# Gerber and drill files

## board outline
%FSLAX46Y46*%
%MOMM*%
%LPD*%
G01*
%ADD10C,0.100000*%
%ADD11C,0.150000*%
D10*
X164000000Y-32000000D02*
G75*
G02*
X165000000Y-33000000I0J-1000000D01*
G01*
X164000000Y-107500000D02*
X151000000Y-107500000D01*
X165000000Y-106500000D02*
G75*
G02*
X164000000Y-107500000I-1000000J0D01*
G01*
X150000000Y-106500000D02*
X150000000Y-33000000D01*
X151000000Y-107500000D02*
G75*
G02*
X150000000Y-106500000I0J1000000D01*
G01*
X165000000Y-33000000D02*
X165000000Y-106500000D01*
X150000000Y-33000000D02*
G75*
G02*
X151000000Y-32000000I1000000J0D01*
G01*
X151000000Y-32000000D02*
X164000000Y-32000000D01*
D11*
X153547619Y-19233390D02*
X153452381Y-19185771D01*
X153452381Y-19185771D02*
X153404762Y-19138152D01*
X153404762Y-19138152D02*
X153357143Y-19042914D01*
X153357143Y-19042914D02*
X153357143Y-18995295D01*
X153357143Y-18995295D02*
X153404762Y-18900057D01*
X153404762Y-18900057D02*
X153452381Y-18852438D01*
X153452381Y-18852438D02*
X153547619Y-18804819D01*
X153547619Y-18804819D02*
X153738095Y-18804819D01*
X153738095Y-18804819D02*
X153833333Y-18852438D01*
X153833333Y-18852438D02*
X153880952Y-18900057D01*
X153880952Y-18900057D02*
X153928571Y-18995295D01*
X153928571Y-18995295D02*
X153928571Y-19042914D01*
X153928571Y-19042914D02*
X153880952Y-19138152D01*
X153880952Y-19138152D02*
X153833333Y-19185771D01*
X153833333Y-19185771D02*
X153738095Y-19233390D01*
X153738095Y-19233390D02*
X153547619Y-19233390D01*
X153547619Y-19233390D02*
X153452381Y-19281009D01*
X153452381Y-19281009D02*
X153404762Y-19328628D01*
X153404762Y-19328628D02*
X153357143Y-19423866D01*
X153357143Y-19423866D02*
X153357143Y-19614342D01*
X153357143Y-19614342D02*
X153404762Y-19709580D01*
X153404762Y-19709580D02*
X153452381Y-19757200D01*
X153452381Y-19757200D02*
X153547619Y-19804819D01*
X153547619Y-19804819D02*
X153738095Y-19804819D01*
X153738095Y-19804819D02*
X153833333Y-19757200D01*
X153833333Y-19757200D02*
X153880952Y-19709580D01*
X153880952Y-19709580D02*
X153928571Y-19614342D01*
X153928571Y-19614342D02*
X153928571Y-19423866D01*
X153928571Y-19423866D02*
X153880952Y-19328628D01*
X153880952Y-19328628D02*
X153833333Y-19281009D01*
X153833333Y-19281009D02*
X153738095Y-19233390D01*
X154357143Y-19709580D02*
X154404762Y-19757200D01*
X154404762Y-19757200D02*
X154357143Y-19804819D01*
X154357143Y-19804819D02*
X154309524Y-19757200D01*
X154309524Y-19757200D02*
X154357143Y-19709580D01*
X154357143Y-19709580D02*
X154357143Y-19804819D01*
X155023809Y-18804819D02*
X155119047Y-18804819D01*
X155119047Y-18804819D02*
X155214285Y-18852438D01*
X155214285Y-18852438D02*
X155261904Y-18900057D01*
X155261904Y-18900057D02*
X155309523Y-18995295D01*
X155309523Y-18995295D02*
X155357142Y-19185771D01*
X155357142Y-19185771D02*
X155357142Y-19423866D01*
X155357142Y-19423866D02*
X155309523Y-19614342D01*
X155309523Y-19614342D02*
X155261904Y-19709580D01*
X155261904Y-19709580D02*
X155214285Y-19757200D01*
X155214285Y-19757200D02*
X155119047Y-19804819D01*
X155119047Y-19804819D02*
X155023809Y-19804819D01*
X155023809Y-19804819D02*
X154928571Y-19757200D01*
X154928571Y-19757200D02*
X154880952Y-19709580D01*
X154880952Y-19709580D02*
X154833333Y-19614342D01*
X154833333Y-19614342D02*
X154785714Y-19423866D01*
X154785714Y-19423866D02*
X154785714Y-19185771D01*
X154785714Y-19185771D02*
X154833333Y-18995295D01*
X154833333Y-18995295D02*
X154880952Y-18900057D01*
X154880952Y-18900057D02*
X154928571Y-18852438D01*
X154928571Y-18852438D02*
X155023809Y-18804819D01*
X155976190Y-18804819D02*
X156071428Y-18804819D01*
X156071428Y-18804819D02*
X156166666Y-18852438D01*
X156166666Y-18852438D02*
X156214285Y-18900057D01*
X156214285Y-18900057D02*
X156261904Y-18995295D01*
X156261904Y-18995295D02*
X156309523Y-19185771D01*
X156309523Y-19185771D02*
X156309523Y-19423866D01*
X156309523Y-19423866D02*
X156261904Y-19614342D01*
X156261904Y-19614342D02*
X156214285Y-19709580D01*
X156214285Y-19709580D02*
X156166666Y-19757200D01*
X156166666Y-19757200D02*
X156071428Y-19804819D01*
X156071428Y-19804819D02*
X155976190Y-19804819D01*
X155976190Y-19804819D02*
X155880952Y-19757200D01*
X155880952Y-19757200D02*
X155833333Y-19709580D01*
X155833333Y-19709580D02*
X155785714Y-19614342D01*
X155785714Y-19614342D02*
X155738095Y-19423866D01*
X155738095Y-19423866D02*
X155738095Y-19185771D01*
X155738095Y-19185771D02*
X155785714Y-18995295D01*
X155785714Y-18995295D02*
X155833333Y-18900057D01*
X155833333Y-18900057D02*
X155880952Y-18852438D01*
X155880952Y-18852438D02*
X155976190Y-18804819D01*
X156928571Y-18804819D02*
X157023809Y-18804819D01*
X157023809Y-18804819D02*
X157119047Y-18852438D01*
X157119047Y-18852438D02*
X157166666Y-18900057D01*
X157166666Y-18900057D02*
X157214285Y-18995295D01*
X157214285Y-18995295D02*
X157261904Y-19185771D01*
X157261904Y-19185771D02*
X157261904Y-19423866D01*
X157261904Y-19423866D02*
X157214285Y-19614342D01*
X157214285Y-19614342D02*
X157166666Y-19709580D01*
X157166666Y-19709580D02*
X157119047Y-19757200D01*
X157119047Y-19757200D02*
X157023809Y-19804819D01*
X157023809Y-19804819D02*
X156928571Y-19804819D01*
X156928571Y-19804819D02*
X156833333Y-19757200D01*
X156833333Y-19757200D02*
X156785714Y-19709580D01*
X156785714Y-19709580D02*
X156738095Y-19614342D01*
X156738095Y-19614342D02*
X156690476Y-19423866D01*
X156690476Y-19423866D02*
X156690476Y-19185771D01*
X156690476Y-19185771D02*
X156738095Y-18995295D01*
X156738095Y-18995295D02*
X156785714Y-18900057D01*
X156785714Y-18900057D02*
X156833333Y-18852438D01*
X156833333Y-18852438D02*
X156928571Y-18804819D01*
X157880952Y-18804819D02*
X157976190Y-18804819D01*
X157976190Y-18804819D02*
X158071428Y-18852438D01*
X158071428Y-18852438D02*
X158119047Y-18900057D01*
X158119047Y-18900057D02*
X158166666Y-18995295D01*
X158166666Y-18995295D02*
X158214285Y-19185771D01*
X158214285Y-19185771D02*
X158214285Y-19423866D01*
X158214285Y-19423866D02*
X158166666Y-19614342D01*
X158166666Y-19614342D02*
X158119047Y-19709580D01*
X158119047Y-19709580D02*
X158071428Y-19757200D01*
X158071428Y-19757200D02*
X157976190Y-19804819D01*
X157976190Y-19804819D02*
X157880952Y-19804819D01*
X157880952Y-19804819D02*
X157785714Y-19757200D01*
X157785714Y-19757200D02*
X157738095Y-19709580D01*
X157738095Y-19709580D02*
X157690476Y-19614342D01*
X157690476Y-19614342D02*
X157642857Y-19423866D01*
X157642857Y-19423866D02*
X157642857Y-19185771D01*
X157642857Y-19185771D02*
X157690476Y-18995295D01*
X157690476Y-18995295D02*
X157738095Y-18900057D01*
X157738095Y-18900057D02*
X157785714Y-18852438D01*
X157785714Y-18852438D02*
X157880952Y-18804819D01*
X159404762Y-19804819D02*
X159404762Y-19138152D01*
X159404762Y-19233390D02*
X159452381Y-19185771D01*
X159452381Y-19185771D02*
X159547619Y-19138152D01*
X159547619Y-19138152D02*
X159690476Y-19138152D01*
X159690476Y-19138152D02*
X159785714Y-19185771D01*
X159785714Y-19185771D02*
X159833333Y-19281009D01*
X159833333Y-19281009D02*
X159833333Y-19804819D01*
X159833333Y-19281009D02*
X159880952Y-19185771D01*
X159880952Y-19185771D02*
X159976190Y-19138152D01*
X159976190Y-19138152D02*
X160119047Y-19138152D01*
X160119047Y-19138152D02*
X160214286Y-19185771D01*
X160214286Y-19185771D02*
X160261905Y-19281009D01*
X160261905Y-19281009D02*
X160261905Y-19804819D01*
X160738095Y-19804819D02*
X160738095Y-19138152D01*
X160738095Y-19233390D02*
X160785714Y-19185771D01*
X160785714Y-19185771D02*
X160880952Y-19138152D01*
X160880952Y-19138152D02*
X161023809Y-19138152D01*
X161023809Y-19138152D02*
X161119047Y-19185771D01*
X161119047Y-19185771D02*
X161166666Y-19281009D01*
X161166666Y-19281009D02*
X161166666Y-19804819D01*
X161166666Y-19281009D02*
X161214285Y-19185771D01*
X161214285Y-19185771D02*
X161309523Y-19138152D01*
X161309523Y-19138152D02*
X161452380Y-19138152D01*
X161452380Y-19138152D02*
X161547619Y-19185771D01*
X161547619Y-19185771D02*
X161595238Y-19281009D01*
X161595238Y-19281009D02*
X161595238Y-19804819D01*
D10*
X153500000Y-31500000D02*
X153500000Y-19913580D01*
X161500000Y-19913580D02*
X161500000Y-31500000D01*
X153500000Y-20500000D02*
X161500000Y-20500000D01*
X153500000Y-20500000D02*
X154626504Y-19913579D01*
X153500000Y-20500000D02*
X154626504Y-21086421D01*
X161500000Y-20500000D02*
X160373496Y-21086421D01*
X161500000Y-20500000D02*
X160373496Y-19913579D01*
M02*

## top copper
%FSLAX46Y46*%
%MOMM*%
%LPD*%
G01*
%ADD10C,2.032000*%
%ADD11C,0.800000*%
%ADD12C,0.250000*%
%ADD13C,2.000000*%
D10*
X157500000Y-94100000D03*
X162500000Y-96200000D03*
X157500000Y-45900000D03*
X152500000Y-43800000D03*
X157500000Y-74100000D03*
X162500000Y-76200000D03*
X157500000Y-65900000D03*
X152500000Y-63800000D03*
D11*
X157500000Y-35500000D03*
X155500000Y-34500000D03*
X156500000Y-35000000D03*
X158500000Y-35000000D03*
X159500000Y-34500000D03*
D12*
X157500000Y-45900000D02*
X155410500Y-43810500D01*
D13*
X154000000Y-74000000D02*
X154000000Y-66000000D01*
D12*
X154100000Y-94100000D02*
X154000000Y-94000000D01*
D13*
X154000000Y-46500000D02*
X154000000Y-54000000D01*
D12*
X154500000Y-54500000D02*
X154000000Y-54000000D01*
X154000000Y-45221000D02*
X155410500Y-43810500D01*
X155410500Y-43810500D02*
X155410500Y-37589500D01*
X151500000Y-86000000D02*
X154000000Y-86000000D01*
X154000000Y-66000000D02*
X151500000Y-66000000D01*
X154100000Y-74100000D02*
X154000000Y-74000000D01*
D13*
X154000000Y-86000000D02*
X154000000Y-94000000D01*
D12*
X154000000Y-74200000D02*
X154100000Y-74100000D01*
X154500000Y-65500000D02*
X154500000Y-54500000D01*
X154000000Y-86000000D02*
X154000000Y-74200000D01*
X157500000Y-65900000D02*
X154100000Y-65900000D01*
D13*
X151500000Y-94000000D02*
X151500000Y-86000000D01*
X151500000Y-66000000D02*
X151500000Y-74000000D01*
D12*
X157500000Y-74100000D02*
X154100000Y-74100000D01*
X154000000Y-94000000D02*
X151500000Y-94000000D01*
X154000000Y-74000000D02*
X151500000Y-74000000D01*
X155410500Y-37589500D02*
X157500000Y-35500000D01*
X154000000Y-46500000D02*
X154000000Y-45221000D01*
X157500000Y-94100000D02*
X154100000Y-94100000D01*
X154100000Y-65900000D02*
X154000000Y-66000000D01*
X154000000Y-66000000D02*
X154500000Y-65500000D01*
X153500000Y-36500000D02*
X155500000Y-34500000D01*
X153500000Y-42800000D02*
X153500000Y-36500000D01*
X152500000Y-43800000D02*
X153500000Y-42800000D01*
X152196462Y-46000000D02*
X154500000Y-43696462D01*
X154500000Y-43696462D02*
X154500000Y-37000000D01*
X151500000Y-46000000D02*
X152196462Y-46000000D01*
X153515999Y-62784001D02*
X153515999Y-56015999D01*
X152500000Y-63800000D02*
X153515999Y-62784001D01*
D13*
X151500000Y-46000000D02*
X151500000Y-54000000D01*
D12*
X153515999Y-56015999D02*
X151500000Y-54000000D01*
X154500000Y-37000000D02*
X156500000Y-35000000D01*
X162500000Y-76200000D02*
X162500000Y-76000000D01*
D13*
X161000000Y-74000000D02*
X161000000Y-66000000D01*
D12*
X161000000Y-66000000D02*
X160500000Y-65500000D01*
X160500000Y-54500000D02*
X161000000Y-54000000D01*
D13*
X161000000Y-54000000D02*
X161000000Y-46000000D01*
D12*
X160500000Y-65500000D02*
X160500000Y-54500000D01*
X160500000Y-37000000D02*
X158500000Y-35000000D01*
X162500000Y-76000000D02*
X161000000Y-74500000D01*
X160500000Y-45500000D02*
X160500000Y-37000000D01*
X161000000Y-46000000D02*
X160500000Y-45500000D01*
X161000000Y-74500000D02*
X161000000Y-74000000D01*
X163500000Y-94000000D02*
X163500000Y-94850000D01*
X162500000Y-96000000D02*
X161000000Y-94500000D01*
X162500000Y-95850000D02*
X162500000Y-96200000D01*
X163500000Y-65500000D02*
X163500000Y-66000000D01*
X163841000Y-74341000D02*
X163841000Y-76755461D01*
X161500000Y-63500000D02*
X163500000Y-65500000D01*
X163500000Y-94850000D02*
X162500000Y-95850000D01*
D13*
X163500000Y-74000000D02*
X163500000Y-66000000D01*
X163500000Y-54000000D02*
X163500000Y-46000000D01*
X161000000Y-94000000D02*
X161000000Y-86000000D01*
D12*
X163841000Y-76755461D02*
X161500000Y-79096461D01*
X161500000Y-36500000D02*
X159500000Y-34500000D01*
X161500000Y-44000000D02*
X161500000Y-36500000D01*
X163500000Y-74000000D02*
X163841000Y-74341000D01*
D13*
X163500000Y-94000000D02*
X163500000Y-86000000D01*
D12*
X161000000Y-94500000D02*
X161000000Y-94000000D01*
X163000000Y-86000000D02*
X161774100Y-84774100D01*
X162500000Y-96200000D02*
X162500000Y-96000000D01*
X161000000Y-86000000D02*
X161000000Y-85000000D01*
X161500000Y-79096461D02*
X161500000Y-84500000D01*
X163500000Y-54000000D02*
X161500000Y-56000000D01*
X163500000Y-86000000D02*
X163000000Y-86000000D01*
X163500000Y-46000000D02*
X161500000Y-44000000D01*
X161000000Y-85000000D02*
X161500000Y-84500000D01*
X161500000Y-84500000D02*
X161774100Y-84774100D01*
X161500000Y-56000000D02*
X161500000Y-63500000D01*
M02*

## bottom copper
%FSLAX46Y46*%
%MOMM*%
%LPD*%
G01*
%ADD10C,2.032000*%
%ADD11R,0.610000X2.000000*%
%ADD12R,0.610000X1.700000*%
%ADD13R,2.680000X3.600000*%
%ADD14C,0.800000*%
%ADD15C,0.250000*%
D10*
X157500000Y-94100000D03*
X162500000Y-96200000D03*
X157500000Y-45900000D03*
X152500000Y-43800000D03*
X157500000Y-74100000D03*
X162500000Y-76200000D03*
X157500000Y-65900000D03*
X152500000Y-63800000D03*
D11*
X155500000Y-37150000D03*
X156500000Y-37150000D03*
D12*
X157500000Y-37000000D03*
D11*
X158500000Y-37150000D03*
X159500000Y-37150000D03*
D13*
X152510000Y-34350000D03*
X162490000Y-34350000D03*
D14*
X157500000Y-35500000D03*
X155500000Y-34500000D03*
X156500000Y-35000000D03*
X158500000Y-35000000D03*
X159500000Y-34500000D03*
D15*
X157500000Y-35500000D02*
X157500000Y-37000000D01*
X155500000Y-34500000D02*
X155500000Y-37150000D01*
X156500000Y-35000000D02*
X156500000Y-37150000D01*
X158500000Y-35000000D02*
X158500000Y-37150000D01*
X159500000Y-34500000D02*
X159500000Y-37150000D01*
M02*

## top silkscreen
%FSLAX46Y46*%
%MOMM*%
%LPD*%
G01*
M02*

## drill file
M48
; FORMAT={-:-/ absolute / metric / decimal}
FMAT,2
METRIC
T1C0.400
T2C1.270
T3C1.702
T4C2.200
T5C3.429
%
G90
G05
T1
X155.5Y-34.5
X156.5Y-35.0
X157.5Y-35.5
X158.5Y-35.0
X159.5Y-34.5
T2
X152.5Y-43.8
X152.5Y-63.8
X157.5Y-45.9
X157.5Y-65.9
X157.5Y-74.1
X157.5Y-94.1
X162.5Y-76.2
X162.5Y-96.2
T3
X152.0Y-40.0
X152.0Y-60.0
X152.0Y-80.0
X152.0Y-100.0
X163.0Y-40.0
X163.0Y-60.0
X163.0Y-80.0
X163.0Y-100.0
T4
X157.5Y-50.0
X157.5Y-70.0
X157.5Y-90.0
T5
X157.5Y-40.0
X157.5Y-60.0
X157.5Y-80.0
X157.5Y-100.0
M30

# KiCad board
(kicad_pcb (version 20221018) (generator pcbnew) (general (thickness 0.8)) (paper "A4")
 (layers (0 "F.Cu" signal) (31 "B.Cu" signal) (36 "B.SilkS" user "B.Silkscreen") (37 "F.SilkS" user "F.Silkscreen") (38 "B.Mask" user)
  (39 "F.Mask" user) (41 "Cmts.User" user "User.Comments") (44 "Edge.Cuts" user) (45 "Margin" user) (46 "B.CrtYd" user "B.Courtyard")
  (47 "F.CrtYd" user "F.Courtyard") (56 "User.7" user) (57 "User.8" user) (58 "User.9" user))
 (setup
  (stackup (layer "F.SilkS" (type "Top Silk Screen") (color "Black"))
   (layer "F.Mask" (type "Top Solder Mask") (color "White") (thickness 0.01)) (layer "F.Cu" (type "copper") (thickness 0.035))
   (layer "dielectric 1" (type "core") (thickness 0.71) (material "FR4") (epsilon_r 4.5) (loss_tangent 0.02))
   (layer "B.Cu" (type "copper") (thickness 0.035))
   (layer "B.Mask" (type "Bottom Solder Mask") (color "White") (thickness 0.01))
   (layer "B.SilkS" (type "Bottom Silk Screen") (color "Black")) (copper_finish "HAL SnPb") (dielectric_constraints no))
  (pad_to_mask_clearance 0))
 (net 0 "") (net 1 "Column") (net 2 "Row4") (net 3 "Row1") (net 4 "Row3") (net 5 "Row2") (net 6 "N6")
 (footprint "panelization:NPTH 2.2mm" (layer "F.Cu") (at 157.5 90)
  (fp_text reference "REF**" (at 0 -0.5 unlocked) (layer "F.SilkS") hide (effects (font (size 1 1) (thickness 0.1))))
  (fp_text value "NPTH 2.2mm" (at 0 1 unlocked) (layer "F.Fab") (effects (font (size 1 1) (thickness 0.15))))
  (pad "" np_thru_hole circle (at 0 0) (size 2.2 2.2) (drill 2.2) (layers "F&B.Cu" "*.Mask")))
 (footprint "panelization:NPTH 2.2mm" (layer "F.Cu") (at 157.5 50)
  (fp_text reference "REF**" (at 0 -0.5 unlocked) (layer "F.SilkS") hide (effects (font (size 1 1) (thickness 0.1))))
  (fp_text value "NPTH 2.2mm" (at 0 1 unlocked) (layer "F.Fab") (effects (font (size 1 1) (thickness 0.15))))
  (pad "" np_thru_hole circle (at 0 0) (size 2.2 2.2) (drill 2.2) (layers "F&B.Cu" "*.Mask")))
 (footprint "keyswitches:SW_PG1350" (layer "F.Cu") (at 157.5 100 180)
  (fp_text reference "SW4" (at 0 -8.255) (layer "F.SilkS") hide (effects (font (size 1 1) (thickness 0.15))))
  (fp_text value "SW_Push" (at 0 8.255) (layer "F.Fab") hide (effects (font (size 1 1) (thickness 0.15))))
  (pad "" np_thru_hole circle (at -5.5 0 180) (size 1.7018 1.7018) (drill 1.7018) (layers "*.Cu" "*.Mask"))
  (pad "" np_thru_hole circle (at 0 0 180) (size 3.429 3.429) (drill 3.429) (layers "*.Cu" "*.Mask"))
  (pad "" np_thru_hole circle (at 5.5 0 180) (size 1.7018 1.7018) (drill 1.7018) (layers "*.Cu" "*.Mask"))
  (pad "1" thru_hole circle (at 0 5.9 180) (size 2.032 2.032) (drill 1.27) (layers "*.Cu" "*.Mask") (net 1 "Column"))
  (pad "2" thru_hole circle (at -5 3.8 180) (size 2.032 2.032) (drill 1.27) (layers "*.Cu" "*.Mask") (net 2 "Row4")))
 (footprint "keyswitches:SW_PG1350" (layer "F.Cu") (at 157.5 40)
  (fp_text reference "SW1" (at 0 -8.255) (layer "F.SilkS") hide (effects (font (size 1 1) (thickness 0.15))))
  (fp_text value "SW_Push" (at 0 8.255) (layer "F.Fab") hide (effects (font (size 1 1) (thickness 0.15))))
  (pad "" np_thru_hole circle (at -5.5 0) (size 1.7018 1.7018) (drill 1.7018) (layers "*.Cu" "*.Mask"))
  (pad "" np_thru_hole circle (at 0 0) (size 3.429 3.429) (drill 3.429) (layers "*.Cu" "*.Mask"))
  (pad "" np_thru_hole circle (at 5.5 0) (size 1.7018 1.7018) (drill 1.7018) (layers "*.Cu" "*.Mask"))
  (pad "1" thru_hole circle (at 0 5.9) (size 2.032 2.032) (drill 1.27) (layers "*.Cu" "*.Mask") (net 1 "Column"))
  (pad "2" thru_hole circle (at -5 3.8) (size 2.032 2.032) (drill 1.27) (layers "*.Cu" "*.Mask") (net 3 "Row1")))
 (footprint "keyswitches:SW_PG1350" (layer "F.Cu") (at 157.5 80 180)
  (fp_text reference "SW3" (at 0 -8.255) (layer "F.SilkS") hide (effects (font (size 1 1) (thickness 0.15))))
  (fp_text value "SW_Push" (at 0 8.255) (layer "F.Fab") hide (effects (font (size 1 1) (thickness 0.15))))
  (pad "" np_thru_hole circle (at -5.5 0 180) (size 1.7018 1.7018) (drill 1.7018) (layers "*.Cu" "*.Mask"))
  (pad "" np_thru_hole circle (at 0 0 180) (size 3.429 3.429) (drill 3.429) (layers "*.Cu" "*.Mask"))
  (pad "" np_thru_hole circle (at 5.5 0 180) (size 1.7018 1.7018) (drill 1.7018) (layers "*.Cu" "*.Mask"))
  (pad "1" thru_hole circle (at 0 5.9 180) (size 2.032 2.032) (drill 1.27) (layers "*.Cu" "*.Mask") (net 1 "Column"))
  (pad "2" thru_hole circle (at -5 3.8 180) (size 2.032 2.032) (drill 1.27) (layers "*.Cu" "*.Mask") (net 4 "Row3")))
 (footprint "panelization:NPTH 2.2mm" (layer "F.Cu") (at 157.5 70)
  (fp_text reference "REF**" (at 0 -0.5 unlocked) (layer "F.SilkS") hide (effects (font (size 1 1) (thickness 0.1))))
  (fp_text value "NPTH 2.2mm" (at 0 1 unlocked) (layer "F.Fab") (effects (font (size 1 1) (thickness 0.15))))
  (pad "" np_thru_hole circle (at 0 0) (size 2.2 2.2) (drill 2.2) (layers "F&B.Cu" "*.Mask")))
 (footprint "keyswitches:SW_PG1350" (layer "F.Cu") (at 157.5 60)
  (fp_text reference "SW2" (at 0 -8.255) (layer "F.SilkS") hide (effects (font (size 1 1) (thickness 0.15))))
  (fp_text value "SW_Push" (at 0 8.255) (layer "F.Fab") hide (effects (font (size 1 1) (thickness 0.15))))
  (pad "" np_thru_hole circle (at -5.5 0) (size 1.7018 1.7018) (drill 1.7018) (layers "*.Cu" "*.Mask"))
  (pad "" np_thru_hole circle (at 0 0) (size 3.429 3.429) (drill 3.429) (layers "*.Cu" "*.Mask"))
  (pad "" np_thru_hole circle (at 5.5 0) (size 1.7018 1.7018) (drill 1.7018) (layers "*.Cu" "*.Mask"))
  (pad "1" thru_hole circle (at 0 5.9) (size 2.032 2.032) (drill 1.27) (layers "*.Cu" "*.Mask") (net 1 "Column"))
  (pad "2" thru_hole circle (at -5 3.8) (size 2.032 2.032) (drill 1.27) (layers "*.Cu" "*.Mask") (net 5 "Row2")))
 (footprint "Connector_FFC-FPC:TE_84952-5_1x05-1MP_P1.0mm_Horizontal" (layer "B.Cu") (at 157.5 35.35)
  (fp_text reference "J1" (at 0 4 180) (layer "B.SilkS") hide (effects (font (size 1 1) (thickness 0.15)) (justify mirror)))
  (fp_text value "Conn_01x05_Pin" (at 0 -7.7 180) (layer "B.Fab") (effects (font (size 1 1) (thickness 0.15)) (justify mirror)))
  (pad "1" smd rect (at -2 1.8) (size 0.61 2) (layers "B.Cu" "B.Paste" "B.Mask") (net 3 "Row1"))
  (pad "2" smd rect (at -1 1.8) (size 0.61 2) (layers "B.Cu" "B.Paste" "B.Mask") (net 5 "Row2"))
  (pad "3" smd rect (at 0 1.65) (size 0.61 1.7) (layers "B.Cu" "B.Paste" "B.Mask") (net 1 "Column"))
  (pad "4" smd rect (at 1 1.8) (size 0.61 2) (layers "B.Cu" "B.Paste" "B.Mask") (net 4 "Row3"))
  (pad "5" smd rect (at 2 1.8) (size 0.61 2) (layers "B.Cu" "B.Paste" "B.Mask") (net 2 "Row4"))
  (pad "MP" smd rect (at -4.99 -1) (size 2.68 3.6) (layers "B.Cu" "B.Paste" "B.Mask") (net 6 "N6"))
  (pad "MP" smd rect (at 4.99 -1) (size 2.68 3.6) (layers "B.Cu" "B.Paste" "B.Mask") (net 6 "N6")))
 (gr_arc (start 164 32) (mid 164.707107 32.292893) (end 165 33) (stroke (width 0.1) (type default)) (layer "Edge.Cuts"))
 (gr_line (start 164 107.5) (end 151 107.5) (stroke (width 0.1) (type default)) (layer "Edge.Cuts"))
 (gr_arc (start 165 106.5) (mid 164.707107 107.207107) (end 164 107.5) (stroke (width 0.1) (type default)) (layer "Edge.Cuts"))
 (gr_line (start 150 106.5) (end 150 33) (stroke (width 0.1) (type default)) (layer "Edge.Cuts"))
 (gr_arc (start 151 107.5) (mid 150.292893 107.207107) (end 150 106.5) (stroke (width 0.1) (type default)) (layer "Edge.Cuts"))
 (gr_line (start 165 33) (end 165 106.5) (stroke (width 0.1) (type default)) (layer "Edge.Cuts"))
 (gr_arc (start 150 33) (mid 150.292893 32.292893) (end 151 32) (stroke (width 0.1) (type default)) (layer "Edge.Cuts"))
 (gr_line (start 151 32) (end 164 32) (stroke (width 0.1) (type default)) (layer "Edge.Cuts"))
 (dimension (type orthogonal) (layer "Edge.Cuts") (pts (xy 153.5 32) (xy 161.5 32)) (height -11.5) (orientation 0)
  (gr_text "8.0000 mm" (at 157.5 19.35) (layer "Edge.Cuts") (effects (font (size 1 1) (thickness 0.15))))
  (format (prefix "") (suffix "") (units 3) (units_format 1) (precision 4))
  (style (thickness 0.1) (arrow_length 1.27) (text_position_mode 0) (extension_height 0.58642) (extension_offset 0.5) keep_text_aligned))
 (segment (start 157.5 45.9) (end 155.4105 43.8105) (width 0.25) (layer "F.Cu") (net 1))
 (segment (start 154 74) (end 154 66) (width 2) (layer "F.Cu") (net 1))
 (segment (start 154.1 94.1) (end 154 94) (width 0.25) (layer "F.Cu") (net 1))
 (segment (start 154 46.5) (end 154 54) (width 2) (layer "F.Cu") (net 1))
 (segment (start 154.5 54.5) (end 154 54) (width 0.25) (layer "F.Cu") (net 1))
 (segment (start 154 45.221) (end 155.4105 43.8105) (width 0.25) (layer "F.Cu") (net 1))
 (segment (start 155.4105 43.8105) (end 155.4105 37.5895) (width 0.25) (layer "F.Cu") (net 1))
 (segment (start 151.5 86) (end 154 86) (width 0.25) (layer "F.Cu") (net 1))
 (segment (start 154 66) (end 151.5 66) (width 0.25) (layer "F.Cu") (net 1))
 (segment (start 154.1 74.1) (end 154 74) (width 0.25) (layer "F.Cu") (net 1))
 (segment (start 154 86) (end 154 94) (width 2) (layer "F.Cu") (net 1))
 (segment (start 154 74.2) (end 154.1 74.1) (width 0.25) (layer "F.Cu") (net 1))
 (segment (start 154.5 65.5) (end 154.5 54.5) (width 0.25) (layer "F.Cu") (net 1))
 (segment (start 154 86) (end 154 74.2) (width 0.25) (layer "F.Cu") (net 1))
 (segment (start 157.5 65.9) (end 154.1 65.9) (width 0.25) (layer "F.Cu") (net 1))
 (segment (start 151.5 94) (end 151.5 86) (width 2) (layer "F.Cu") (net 1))
 (segment (start 151.5 66) (end 151.5 74) (width 2) (layer "F.Cu") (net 1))
 (segment (start 157.5 74.1) (end 154.1 74.1) (width 0.25) (layer "F.Cu") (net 1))
 (segment (start 154 94) (end 151.5 94) (width 0.25) (layer "F.Cu") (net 1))
 (segment (start 154 74) (end 151.5 74) (width 0.25) (layer "F.Cu") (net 1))
 (segment (start 155.4105 37.5895) (end 157.5 35.5) (width 0.25) (layer "F.Cu") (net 1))
 (segment (start 154 46.5) (end 154 45.221) (width 0.25) (layer "F.Cu") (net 1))
 (segment (start 157.5 94.1) (end 154.1 94.1) (width 0.25) (layer "F.Cu") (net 1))
 (segment (start 154.1 65.9) (end 154 66) (width 0.25) (layer "F.Cu") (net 1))
 (segment (start 154 66) (end 154.5 65.5) (width 0.25) (layer "F.Cu") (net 1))
 (via (at 157.5 35.5) (size 0.8) (drill 0.4) (layers "F.Cu" "B.Cu") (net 1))
 (segment (start 157.5 35.5) (end 157.5 37) (width 0.25) (layer "B.Cu") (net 1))
 (segment (start 153.5 36.5) (end 155.5 34.5) (width 0.25) (layer "F.Cu") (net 3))
 (segment (start 153.5 42.8) (end 153.5 36.5) (width 0.25) (layer "F.Cu") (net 3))
 (segment (start 152.5 43.8) (end 153.5 42.8) (width 0.25) (layer "F.Cu") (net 3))
 (via (at 155.5 34.5) (size 0.8) (drill 0.4) (layers "F.Cu" "B.Cu") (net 3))
 (segment (start 155.5 34.5) (end 155.5 37.15) (width 0.25) (layer "B.Cu") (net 3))
 (segment (start 152.196462 46) (end 154.5 43.696462) (width 0.25) (layer "F.Cu") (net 5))
 (segment (start 154.5 43.696462) (end 154.5 37) (width 0.25) (layer "F.Cu") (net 5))
 (segment (start 151.5 46) (end 152.196462 46) (width 0.25) (layer "F.Cu") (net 5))
 (segment (start 153.515999 62.784001) (end 153.515999 56.015999) (width 0.25) (layer "F.Cu") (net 5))
 (segment (start 152.5 63.8) (end 153.515999 62.784001) (width 0.25) (layer "F.Cu") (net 5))
 (segment (start 151.5 46) (end 151.5 54) (width 2) (layer "F.Cu") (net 5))
 (segment (start 153.515999 56.015999) (end 151.5 54) (width 0.25) (layer "F.Cu") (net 5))
 (segment (start 154.5 37) (end 156.5 35) (width 0.25) (layer "F.Cu") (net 5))
 (via (at 156.5 35) (size 0.8) (drill 0.4) (layers "F.Cu" "B.Cu") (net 5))
 (segment (start 156.5 35) (end 156.5 37.15) (width 0.25) (layer "B.Cu") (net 5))
 (segment (start 162.5 76.2) (end 162.5 76) (width 0.25) (layer "F.Cu") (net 4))
 (segment (start 161 74) (end 161 66) (width 2) (layer "F.Cu") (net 4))
 (segment (start 161 66) (end 160.5 65.5) (width 0.25) (layer "F.Cu") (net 4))
 (segment (start 160.5 54.5) (end 161 54) (width 0.25) (layer "F.Cu") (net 4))
 (segment (start 161 54) (end 161 46) (width 2) (layer "F.Cu") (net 4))
 (segment (start 160.5 65.5) (end 160.5 54.5) (width 0.25) (layer "F.Cu") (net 4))
 (segment (start 160.5 37) (end 158.5 35) (width 0.25) (layer "F.Cu") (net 4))
 (segment (start 162.5 76) (end 161 74.5) (width 0.25) (layer "F.Cu") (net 4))
 (segment (start 160.5 45.5) (end 160.5 37) (width 0.25) (layer "F.Cu") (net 4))
 (segment (start 161 46) (end 160.5 45.5) (width 0.25) (layer "F.Cu") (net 4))
 (segment (start 161 74.5) (end 161 74) (width 0.25) (layer "F.Cu") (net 4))
 (via (at 158.5 35) (size 0.8) (drill 0.4) (layers "F.Cu" "B.Cu") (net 4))
 (segment (start 158.5 35) (end 158.5 37.15) (width 0.25) (layer "B.Cu") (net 4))
 (segment (start 163.5 94) (end 163.5 94.85) (width 0.25) (layer "F.Cu") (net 2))
 (segment (start 162.5 96) (end 161 94.5) (width 0.25) (layer "F.Cu") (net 2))
 (segment (start 162.5 95.85) (end 162.5 96.2) (width 0.25) (layer "F.Cu") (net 2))
 (segment (start 163.5 65.5) (end 163.5 66) (width 0.25) (layer "F.Cu") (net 2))
 (segment (start 163.841 74.341) (end 163.841 76.755461) (width 0.25) (layer "F.Cu") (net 2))
 (segment (start 161.5 63.5) (end 163.5 65.5) (width 0.25) (layer "F.Cu") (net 2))
 (segment (start 163.5 94.85) (end 162.5 95.85) (width 0.25) (layer "F.Cu") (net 2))
 (segment (start 163.5 74) (end 163.5 66) (width 2) (layer "F.Cu") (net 2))
 (segment (start 163.5 54) (end 163.5 46) (width 2) (layer "F.Cu") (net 2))
 (segment (start 161 94) (end 161 86) (width 2) (layer "F.Cu") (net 2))
 (segment (start 163.841 76.755461) (end 161.5 79.096461) (width 0.25) (layer "F.Cu") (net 2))
 (segment (start 161.5 36.5) (end 159.5 34.5) (width 0.25) (layer "F.Cu") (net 2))
 (segment (start 161.5 44) (end 161.5 36.5) (width 0.25) (layer "F.Cu") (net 2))
 (segment (start 163.5 74) (end 163.841 74.341) (width 0.25) (layer "F.Cu") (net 2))
 (segment (start 163.5 94) (end 163.5 86) (width 2) (layer "F.Cu") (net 2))
 (segment (start 161 94.5) (end 161 94) (width 0.25) (layer "F.Cu") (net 2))
 (segment (start 163 86) (end 161.7741 84.7741) (width 0.25) (layer "F.Cu") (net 2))
 (segment (start 162.5 96.2) (end 162.5 96) (width 0.25) (layer "F.Cu") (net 2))
 (segment (start 161 86) (end 161 85) (width 0.25) (layer "F.Cu") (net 2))
 (segment (start 161.5 79.096461) (end 161.5 84.5) (width 0.25) (layer "F.Cu") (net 2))
 (segment (start 163.5 54) (end 161.5 56) (width 0.25) (layer "F.Cu") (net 2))
 (segment (start 163.5 86) (end 163 86) (width 0.25) (layer "F.Cu") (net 2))
 (segment (start 163.5 46) (end 161.5 44) (width 0.25) (layer "F.Cu") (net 2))
 (segment (start 161 85) (end 161.5 84.5) (width 0.25) (layer "F.Cu") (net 2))
 (segment (start 161.5 84.5) (end 161.7741 84.7741) (width 0.25) (layer "F.Cu") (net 2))
 (segment (start 161.5 56) (end 161.5 63.5) (width 0.25) (layer "F.Cu") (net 2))
 (via (at 159.5 34.5) (size 0.8) (drill 0.4) (layers "F.Cu" "B.Cu") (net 2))
 (segment (start 159.5 34.5) (end 159.5 37.15) (width 0.25) (layer "B.Cu") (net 2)))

